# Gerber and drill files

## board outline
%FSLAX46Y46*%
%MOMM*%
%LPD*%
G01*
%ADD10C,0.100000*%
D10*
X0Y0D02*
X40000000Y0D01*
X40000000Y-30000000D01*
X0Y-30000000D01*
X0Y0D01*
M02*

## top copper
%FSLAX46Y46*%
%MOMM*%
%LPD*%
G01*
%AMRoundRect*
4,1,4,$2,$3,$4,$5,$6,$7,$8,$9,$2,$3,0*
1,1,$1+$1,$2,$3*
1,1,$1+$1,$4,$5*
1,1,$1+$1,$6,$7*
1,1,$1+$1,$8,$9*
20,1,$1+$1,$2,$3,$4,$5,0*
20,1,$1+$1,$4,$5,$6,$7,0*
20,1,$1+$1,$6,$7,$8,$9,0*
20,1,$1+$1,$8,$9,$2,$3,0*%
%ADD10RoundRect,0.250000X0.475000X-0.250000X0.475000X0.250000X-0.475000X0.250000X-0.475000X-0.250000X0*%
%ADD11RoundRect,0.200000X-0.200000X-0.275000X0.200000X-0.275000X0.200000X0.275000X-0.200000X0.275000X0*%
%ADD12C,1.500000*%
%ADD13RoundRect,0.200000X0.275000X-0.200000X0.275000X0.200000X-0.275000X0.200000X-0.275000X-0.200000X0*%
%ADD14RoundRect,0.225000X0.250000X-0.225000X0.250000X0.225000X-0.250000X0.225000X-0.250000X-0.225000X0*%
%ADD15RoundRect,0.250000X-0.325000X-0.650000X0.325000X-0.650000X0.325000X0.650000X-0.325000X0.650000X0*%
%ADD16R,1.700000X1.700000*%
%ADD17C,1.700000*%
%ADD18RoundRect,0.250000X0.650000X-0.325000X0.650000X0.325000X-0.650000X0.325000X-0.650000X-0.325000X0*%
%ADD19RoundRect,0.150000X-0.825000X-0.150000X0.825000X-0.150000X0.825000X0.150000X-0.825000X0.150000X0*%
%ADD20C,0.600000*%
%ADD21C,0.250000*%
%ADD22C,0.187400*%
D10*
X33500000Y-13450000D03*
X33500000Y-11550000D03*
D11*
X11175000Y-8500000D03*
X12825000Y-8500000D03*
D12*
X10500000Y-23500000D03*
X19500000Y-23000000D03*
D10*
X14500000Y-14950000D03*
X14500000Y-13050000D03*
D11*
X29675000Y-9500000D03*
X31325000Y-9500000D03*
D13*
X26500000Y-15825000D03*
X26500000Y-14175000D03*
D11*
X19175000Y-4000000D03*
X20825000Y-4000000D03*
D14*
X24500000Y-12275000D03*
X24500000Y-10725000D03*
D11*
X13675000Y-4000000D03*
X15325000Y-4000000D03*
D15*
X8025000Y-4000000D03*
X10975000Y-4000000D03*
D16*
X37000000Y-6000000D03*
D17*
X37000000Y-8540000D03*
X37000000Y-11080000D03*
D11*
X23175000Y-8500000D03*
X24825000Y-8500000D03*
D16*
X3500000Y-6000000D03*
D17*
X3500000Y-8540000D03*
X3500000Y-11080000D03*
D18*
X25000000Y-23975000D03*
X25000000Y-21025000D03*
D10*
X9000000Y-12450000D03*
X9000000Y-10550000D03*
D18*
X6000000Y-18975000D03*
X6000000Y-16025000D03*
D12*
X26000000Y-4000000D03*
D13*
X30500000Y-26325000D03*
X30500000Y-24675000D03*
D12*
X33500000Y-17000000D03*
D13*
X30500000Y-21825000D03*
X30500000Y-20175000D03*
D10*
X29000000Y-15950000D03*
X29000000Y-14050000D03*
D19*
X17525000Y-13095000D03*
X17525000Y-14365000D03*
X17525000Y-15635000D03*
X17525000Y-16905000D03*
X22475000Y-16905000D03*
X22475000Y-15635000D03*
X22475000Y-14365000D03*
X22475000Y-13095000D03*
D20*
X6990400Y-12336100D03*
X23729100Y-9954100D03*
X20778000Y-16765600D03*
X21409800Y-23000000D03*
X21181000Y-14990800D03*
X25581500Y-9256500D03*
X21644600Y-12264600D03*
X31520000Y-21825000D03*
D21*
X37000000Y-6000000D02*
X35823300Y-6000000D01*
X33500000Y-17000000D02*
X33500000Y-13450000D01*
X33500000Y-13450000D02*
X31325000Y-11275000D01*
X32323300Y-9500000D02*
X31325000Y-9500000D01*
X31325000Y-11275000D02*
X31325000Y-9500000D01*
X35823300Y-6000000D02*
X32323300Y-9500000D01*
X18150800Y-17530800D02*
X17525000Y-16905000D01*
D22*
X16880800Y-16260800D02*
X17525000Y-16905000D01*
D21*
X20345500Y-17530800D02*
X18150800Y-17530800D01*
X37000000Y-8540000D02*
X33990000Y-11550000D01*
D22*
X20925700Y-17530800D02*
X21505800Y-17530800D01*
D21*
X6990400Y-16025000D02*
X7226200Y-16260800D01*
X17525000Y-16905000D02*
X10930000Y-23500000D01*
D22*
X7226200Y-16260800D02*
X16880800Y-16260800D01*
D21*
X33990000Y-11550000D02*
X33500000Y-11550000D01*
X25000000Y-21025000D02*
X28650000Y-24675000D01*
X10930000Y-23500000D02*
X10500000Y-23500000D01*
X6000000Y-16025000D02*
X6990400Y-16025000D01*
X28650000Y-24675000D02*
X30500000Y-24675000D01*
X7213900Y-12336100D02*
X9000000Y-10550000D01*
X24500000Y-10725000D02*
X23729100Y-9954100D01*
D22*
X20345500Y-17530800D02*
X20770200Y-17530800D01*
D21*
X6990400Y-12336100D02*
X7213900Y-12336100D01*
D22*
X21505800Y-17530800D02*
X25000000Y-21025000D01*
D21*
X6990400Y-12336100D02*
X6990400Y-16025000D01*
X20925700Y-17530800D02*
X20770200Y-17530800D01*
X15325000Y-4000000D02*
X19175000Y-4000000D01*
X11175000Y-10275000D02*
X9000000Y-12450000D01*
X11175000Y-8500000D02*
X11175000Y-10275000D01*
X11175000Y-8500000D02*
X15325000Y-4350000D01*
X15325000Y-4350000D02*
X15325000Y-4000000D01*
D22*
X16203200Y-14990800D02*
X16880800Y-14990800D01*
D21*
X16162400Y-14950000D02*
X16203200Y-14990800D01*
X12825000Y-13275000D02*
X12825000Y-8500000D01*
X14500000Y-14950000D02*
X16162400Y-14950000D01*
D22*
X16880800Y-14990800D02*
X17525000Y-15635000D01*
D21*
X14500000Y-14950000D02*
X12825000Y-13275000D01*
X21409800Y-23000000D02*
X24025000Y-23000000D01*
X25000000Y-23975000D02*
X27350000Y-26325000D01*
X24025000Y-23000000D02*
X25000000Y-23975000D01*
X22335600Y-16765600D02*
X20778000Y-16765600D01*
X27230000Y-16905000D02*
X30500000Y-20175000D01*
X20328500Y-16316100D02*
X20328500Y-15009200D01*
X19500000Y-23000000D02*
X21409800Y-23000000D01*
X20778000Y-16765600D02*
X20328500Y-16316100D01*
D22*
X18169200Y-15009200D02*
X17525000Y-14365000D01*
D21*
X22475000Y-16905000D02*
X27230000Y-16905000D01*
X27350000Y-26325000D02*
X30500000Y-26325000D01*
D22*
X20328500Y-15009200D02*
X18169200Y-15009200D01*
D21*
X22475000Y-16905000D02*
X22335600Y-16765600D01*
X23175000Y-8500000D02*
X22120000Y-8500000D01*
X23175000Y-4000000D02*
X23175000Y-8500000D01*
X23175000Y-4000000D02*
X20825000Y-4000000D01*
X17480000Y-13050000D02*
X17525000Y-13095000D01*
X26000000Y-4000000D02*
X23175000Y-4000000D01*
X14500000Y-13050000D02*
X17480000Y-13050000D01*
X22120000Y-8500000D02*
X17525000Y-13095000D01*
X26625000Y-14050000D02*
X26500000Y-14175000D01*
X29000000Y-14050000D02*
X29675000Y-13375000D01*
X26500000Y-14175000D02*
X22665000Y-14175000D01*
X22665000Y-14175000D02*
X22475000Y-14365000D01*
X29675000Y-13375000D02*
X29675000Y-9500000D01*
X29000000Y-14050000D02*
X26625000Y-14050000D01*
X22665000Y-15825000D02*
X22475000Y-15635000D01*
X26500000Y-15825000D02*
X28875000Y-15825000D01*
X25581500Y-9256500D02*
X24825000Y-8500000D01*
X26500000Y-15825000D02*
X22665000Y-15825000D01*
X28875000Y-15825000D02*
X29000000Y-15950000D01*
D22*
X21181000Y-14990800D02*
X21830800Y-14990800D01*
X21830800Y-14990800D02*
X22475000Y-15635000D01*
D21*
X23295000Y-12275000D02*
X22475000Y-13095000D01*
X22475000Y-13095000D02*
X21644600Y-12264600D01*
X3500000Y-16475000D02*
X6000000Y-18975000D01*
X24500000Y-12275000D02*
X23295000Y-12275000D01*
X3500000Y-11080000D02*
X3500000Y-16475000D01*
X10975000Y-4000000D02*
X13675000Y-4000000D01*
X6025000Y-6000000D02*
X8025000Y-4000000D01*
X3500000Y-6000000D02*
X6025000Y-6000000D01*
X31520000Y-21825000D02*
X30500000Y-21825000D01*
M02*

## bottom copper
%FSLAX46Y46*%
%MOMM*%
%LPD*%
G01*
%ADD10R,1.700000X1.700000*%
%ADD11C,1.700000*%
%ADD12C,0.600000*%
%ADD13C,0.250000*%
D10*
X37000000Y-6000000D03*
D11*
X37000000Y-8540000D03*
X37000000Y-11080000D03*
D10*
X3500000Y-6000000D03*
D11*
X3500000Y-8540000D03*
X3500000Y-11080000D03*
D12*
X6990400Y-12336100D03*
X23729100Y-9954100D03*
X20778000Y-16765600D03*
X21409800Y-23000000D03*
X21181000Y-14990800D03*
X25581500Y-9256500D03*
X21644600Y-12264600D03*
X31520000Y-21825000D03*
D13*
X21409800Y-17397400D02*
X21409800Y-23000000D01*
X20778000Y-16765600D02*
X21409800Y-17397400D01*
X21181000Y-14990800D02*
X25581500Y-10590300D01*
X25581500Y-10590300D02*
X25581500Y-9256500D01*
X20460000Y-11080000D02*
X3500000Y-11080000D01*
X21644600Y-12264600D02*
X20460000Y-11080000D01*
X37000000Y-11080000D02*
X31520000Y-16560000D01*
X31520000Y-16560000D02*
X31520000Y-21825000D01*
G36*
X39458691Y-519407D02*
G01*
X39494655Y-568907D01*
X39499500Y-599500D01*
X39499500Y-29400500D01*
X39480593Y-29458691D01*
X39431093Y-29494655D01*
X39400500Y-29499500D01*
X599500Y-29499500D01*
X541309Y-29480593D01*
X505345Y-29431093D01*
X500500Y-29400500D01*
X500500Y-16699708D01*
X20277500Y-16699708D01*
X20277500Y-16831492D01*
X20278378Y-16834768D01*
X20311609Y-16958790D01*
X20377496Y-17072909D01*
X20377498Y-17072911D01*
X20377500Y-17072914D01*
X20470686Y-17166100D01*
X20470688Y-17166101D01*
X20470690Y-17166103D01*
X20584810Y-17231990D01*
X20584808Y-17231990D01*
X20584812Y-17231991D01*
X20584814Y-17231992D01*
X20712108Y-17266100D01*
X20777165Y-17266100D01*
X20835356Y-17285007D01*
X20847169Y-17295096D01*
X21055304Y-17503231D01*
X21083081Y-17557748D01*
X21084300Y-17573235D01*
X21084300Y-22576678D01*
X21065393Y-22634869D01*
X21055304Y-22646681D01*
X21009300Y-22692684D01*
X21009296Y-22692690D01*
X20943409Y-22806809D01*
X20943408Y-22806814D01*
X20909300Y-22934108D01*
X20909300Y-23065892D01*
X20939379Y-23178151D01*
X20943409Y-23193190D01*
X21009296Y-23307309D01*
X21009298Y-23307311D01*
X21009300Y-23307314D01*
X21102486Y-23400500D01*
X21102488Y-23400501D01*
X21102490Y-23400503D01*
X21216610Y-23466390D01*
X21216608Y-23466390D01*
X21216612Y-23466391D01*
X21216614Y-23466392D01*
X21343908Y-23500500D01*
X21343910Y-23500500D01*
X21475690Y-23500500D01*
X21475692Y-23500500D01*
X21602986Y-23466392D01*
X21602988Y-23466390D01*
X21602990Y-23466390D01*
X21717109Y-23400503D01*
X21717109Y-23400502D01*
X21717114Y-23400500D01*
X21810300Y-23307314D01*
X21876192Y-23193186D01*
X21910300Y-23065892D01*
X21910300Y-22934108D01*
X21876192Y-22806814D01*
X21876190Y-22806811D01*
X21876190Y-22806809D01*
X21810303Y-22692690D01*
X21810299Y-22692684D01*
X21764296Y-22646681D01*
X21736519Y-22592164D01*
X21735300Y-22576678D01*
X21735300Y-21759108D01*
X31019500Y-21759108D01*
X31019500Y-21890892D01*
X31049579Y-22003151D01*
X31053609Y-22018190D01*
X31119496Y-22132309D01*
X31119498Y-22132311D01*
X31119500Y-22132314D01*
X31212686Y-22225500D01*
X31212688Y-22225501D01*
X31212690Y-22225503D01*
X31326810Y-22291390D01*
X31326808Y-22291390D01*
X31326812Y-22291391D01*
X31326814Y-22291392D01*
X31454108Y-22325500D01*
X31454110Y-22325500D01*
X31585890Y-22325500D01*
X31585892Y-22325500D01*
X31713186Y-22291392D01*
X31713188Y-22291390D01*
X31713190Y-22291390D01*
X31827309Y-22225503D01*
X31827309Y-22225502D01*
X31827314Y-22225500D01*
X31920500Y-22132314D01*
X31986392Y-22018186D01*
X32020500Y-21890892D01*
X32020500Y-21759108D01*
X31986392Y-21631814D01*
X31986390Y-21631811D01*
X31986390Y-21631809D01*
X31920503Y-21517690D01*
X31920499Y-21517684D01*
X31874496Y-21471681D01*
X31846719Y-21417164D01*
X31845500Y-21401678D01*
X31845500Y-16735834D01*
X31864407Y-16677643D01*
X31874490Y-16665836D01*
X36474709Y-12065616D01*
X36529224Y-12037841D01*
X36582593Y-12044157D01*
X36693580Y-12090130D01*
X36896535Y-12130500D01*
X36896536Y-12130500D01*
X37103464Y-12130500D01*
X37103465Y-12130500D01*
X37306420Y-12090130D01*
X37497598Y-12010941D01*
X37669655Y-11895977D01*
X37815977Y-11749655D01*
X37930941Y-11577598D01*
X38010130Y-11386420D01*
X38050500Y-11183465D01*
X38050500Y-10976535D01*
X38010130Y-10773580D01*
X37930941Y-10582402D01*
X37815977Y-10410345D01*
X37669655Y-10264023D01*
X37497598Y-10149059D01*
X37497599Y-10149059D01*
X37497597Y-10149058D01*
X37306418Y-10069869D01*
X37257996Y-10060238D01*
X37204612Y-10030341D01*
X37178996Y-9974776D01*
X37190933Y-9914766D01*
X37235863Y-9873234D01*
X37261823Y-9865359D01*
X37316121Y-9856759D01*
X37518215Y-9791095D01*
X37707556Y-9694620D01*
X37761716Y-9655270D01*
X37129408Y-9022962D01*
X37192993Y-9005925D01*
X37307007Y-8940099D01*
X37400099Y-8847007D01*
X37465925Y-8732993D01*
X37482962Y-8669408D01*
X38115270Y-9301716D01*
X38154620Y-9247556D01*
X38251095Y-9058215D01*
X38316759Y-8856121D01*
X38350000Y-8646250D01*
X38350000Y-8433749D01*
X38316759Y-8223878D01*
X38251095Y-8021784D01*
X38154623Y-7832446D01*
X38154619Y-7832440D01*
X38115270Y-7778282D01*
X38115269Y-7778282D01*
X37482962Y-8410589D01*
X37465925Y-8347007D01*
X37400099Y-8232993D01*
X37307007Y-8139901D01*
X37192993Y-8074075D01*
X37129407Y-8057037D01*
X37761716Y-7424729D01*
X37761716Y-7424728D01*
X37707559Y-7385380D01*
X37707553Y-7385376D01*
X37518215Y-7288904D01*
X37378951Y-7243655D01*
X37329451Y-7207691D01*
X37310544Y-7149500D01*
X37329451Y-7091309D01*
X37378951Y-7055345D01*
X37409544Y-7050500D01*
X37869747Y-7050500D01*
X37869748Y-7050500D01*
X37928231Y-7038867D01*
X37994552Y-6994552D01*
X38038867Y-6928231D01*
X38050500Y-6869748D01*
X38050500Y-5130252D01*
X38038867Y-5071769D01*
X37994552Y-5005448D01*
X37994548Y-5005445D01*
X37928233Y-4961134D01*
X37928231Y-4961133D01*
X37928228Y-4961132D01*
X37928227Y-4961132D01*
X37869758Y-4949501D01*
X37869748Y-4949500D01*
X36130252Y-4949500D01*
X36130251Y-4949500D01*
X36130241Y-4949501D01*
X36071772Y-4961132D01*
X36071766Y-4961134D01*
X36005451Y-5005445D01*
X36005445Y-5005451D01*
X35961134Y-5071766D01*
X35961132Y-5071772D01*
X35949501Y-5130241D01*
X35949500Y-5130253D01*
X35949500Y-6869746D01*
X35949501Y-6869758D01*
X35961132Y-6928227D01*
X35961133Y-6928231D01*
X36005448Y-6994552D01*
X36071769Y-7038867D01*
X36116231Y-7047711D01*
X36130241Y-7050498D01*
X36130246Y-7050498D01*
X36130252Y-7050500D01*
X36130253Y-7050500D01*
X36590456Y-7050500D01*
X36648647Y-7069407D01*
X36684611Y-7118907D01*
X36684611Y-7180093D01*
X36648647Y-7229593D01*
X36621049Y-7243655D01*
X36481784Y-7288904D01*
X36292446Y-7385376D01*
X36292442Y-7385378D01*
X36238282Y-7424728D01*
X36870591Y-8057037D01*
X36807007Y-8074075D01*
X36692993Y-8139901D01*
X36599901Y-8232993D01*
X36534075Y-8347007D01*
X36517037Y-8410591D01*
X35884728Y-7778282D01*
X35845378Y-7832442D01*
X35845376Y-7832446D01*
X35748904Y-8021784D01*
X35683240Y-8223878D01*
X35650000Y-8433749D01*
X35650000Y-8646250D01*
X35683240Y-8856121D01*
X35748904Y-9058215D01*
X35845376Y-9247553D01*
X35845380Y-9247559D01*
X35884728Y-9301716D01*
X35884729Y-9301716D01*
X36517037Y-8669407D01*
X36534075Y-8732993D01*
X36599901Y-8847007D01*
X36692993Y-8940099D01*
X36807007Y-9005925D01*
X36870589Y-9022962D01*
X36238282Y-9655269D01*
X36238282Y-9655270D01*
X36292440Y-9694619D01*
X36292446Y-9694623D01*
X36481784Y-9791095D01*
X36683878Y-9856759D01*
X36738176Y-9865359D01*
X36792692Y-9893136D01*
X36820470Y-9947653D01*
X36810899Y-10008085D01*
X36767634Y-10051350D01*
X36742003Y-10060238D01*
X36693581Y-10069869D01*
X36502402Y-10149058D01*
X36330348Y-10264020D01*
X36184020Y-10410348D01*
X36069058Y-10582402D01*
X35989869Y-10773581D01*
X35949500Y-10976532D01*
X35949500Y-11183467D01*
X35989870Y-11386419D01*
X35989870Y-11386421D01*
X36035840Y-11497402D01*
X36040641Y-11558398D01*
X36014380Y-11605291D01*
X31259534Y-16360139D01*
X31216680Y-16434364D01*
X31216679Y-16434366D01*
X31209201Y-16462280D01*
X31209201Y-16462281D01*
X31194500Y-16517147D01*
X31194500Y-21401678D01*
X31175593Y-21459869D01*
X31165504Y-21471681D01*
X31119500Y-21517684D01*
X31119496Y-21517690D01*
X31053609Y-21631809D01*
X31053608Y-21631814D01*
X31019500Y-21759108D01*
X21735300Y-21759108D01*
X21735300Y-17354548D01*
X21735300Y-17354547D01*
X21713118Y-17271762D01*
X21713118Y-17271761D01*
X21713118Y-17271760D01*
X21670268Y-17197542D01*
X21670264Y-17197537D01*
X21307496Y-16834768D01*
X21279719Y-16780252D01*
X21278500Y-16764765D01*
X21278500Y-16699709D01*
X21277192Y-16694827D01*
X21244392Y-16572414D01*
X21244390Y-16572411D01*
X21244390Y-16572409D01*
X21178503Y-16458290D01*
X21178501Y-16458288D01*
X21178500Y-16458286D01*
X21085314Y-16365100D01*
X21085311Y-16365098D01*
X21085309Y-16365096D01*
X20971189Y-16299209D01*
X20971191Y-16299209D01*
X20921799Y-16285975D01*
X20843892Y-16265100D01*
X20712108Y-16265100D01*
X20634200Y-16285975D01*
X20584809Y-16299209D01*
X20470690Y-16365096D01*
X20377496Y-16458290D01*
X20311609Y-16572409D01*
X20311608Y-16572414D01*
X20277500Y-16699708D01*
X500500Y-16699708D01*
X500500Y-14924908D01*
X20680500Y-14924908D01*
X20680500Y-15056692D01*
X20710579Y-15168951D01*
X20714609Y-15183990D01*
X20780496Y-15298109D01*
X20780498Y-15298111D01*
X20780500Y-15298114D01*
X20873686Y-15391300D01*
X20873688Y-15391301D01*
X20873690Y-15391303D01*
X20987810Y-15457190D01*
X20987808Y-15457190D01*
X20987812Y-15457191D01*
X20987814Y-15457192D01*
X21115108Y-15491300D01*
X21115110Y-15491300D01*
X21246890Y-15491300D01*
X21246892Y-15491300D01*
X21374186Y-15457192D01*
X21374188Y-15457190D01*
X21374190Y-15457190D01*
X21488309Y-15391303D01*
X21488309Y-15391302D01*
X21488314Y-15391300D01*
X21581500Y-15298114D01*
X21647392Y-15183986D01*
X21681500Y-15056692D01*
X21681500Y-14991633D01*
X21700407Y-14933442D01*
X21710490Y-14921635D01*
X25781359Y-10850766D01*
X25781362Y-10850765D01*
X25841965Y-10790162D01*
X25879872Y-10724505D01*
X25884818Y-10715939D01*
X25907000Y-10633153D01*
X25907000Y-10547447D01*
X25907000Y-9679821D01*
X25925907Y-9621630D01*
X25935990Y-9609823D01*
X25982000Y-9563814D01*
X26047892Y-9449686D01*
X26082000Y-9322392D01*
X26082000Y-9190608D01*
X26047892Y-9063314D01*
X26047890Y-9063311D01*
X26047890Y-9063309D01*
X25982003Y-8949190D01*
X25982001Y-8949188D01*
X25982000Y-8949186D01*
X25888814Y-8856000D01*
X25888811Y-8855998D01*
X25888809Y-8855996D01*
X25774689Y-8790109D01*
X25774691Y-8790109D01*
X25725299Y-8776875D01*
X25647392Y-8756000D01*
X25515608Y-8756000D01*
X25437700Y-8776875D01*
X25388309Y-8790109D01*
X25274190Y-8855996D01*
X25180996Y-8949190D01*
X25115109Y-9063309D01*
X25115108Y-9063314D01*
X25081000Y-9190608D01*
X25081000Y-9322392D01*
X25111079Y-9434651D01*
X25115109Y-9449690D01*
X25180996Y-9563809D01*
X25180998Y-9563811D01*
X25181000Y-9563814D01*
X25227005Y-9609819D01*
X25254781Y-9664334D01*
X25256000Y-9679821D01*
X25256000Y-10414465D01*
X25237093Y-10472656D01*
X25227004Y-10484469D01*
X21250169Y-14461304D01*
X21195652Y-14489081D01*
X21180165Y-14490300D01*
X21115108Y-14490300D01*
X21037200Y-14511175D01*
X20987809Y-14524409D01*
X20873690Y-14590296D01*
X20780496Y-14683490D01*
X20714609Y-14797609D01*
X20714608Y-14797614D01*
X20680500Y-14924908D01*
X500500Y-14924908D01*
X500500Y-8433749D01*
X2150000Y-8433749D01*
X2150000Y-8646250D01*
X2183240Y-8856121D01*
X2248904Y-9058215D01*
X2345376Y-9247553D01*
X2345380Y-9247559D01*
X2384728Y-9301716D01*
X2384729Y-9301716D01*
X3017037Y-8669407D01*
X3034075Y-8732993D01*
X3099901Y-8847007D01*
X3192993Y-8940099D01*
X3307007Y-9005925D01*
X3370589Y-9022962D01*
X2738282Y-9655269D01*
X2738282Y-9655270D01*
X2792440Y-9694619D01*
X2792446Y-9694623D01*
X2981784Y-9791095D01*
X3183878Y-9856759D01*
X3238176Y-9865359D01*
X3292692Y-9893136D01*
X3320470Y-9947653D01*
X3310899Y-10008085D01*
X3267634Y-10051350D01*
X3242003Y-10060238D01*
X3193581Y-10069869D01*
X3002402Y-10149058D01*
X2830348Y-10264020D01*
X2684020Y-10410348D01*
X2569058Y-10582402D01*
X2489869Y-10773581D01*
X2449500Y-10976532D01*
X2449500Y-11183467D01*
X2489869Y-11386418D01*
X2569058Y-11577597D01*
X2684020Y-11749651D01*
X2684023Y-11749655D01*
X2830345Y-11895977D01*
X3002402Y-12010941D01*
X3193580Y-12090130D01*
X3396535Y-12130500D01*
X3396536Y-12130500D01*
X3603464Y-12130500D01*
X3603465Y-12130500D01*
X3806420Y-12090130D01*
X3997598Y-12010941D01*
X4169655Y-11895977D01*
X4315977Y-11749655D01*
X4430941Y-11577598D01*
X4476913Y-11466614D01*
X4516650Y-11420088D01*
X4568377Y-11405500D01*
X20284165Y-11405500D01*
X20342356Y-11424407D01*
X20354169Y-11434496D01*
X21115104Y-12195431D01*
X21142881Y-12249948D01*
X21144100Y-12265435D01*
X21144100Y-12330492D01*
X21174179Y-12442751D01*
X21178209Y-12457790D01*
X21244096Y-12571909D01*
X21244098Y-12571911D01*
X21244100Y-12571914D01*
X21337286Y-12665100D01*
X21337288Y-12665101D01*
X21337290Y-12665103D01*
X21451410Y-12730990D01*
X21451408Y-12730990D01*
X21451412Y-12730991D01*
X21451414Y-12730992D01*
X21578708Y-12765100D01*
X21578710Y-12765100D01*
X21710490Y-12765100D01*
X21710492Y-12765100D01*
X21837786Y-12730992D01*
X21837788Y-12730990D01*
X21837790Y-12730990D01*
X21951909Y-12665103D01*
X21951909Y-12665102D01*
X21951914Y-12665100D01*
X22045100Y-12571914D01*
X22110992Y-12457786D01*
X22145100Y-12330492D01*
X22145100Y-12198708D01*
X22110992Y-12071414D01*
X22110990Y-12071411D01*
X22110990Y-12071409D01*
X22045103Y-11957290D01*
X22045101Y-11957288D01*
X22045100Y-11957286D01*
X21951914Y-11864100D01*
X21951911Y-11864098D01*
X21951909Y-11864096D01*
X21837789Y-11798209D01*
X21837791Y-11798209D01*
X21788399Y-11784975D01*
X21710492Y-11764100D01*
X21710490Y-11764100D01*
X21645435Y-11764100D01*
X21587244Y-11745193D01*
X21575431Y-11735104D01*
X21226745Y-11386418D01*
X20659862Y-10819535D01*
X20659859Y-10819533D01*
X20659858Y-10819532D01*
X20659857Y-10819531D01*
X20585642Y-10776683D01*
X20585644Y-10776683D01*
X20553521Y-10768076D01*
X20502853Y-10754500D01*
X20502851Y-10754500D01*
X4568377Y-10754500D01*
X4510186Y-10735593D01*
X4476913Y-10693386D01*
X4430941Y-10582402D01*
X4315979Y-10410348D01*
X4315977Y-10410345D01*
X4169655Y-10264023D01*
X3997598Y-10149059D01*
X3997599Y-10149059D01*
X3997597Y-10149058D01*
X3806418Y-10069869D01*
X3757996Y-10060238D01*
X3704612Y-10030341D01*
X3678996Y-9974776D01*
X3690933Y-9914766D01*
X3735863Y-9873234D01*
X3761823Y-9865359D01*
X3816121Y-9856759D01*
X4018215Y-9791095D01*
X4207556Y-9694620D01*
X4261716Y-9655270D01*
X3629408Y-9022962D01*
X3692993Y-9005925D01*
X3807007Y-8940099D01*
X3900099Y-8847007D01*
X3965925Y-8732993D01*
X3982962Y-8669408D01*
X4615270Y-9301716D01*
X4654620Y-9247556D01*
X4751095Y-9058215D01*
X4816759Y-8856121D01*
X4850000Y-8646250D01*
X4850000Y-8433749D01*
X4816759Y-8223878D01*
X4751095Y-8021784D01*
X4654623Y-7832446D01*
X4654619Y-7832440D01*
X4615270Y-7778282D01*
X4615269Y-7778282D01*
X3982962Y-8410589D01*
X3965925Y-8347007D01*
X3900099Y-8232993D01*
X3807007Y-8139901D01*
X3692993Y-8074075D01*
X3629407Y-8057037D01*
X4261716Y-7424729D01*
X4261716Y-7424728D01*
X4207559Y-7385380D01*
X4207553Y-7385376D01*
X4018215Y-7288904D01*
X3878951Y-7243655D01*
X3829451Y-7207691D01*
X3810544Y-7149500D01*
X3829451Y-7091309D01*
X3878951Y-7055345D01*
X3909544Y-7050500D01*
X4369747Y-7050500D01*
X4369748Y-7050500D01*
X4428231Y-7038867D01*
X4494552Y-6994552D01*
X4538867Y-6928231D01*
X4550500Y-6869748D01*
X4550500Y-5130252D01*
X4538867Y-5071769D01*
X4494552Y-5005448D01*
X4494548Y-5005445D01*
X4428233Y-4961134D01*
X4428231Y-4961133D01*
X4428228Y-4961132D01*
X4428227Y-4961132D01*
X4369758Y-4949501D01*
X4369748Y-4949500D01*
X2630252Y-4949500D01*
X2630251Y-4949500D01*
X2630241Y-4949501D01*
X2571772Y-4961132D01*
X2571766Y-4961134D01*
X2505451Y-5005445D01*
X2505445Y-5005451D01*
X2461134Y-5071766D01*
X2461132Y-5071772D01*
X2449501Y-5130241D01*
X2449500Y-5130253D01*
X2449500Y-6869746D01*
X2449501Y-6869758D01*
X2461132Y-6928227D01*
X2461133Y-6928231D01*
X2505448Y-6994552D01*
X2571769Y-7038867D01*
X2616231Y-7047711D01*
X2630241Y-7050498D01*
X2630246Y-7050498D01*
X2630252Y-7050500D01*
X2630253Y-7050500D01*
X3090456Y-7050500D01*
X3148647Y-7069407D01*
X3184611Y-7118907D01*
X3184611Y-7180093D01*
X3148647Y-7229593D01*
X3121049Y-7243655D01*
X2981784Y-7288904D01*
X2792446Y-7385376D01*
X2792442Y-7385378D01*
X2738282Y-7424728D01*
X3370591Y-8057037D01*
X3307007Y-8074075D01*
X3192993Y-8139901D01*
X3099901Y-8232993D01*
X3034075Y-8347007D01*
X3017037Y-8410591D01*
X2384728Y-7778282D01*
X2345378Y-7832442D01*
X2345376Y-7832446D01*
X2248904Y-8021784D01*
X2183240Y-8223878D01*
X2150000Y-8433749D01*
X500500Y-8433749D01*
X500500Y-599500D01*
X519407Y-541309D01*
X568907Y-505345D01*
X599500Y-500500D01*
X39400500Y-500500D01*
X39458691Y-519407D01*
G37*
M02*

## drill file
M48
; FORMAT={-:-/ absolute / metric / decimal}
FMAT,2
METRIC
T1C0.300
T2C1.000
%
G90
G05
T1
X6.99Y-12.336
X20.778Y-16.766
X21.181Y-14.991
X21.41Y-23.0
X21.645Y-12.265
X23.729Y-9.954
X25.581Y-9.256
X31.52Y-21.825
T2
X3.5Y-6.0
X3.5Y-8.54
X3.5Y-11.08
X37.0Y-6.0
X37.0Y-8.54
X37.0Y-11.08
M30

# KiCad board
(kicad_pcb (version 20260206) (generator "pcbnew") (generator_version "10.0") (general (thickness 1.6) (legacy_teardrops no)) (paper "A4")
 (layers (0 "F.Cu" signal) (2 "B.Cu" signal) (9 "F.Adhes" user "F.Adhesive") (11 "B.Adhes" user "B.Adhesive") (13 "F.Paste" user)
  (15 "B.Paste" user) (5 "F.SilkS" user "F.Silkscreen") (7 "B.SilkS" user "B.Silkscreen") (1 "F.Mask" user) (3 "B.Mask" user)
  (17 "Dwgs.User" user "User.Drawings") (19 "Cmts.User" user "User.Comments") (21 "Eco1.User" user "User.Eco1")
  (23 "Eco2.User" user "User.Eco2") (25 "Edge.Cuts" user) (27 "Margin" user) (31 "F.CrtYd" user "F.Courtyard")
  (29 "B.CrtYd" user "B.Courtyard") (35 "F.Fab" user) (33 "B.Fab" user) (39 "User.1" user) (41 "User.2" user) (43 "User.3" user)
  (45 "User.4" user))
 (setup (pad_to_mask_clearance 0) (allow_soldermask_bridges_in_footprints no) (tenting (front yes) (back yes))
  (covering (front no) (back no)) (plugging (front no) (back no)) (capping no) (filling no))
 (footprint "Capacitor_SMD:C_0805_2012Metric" (layer "F.Cu") (at 33.5 12.5 90)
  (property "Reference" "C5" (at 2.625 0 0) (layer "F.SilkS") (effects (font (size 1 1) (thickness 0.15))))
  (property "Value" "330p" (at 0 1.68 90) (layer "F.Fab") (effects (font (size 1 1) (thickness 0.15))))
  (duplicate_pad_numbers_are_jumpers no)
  (pad "1" smd roundrect (at -0.95 0 90) (size 1 1.45) (layers "F.Cu" "F.Mask" "F.Paste") (roundrect_rratio 0.25) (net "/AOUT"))
  (pad "2" smd roundrect (at 0.95 0 90) (size 1 1.45) (layers "F.Cu" "F.Mask" "F.Paste") (roundrect_rratio 0.25) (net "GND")))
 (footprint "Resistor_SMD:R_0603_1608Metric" (layer "F.Cu") (at 12 8.5)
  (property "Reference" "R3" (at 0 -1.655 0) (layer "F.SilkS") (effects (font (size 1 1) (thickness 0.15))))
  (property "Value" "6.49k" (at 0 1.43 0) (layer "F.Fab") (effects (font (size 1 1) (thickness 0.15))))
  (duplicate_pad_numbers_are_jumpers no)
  (pad "1" smd roundrect (at -0.825 0) (size 0.8 0.95) (layers "F.Cu" "F.Mask" "F.Paste") (roundrect_rratio 0.25) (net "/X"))
  (pad "2" smd roundrect (at 0.825 0) (size 0.8 0.95) (layers "F.Cu" "F.Mask" "F.Paste") (roundrect_rratio 0.25) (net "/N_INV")))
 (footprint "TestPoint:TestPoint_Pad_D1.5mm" (layer "F.Cu") (at 10.5 23.5)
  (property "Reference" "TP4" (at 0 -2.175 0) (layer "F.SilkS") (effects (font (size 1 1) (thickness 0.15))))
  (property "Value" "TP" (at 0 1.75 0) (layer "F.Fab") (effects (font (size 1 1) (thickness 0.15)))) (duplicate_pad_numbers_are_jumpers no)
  (pad "1" smd circle (at 0 0) (size 1.5 1.5) (layers "F.Cu" "F.Mask") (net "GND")))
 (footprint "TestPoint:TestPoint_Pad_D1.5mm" (layer "F.Cu") (at 19.5 23)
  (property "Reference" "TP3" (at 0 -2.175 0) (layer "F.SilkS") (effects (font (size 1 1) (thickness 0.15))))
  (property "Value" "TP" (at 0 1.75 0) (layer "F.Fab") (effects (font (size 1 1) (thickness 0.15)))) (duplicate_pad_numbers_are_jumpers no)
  (pad "1" smd circle (at 0 0) (size 1.5 1.5) (layers "F.Cu" "F.Mask") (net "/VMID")))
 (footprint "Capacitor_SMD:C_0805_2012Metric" (layer "F.Cu") (at 14.5 14 90)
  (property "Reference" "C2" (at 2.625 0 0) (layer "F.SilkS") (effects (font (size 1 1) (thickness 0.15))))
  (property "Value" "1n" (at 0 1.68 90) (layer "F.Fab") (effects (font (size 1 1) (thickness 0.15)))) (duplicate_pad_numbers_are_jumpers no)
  (pad "1" smd roundrect (at -0.95 0 90) (size 1 1.45) (layers "F.Cu" "F.Mask" "F.Paste") (roundrect_rratio 0.25) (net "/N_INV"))
  (pad "2" smd roundrect (at 0.95 0 90) (size 1 1.45) (layers "F.Cu" "F.Mask" "F.Paste") (roundrect_rratio 0.25) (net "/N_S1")))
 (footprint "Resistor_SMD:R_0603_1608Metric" (layer "F.Cu") (at 30.5 9.5)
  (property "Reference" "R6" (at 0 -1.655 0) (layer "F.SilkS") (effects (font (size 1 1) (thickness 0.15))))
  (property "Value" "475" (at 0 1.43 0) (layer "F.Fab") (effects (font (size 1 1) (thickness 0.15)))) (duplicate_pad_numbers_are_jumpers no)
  (pad "1" smd roundrect (at -0.825 0) (size 0.8 0.95) (layers "F.Cu" "F.Mask" "F.Paste") (roundrect_rratio 0.25) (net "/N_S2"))
  (pad "2" smd roundrect (at 0.825 0) (size 0.8 0.95) (layers "F.Cu" "F.Mask" "F.Paste") (roundrect_rratio 0.25) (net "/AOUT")))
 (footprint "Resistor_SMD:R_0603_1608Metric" (layer "F.Cu") (at 26.5 15 90)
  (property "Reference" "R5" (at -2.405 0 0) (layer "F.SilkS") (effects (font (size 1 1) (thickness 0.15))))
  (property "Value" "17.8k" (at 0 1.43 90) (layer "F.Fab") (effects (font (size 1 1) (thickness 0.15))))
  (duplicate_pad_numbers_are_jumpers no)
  (pad "1" smd roundrect (at -0.825 0 90) (size 0.8 0.95) (layers "F.Cu" "F.Mask" "F.Paste") (roundrect_rratio 0.25) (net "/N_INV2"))
  (pad "2" smd roundrect (at 0.825 0 90) (size 0.8 0.95) (layers "F.Cu" "F.Mask" "F.Paste") (roundrect_rratio 0.25) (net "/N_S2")))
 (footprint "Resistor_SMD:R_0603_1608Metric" (layer "F.Cu") (at 20 4)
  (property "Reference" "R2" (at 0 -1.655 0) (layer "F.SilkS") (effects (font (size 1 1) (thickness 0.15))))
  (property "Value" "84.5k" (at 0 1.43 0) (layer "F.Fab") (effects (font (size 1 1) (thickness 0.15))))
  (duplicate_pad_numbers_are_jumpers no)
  (pad "1" smd roundrect (at -0.825 0) (size 0.8 0.95) (layers "F.Cu" "F.Mask" "F.Paste") (roundrect_rratio 0.25) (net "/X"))
  (pad "2" smd roundrect (at 0.825 0) (size 0.8 0.95) (layers "F.Cu" "F.Mask" "F.Paste") (roundrect_rratio 0.25) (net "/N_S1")))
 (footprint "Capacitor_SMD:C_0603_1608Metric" (layer "F.Cu") (at 24.5 11.5 90)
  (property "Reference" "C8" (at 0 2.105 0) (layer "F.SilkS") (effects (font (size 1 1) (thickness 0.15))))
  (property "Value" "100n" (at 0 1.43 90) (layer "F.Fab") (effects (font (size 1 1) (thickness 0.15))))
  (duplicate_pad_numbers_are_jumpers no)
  (pad "1" smd roundrect (at -0.775 0 90) (size 0.9 0.95) (layers "F.Cu" "F.Mask" "F.Paste") (roundrect_rratio 0.25) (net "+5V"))
  (pad "2" smd roundrect (at 0.775 0 90) (size 0.9 0.95) (layers "F.Cu" "F.Mask" "F.Paste") (roundrect_rratio 0.25) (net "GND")))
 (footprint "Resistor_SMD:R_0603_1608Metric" (layer "F.Cu") (at 14.5 4)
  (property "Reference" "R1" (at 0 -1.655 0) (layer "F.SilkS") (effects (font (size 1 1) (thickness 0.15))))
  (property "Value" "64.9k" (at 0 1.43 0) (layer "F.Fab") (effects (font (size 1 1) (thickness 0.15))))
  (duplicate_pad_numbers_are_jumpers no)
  (pad "1" smd roundrect (at -0.825 0) (size 0.8 0.95) (layers "F.Cu" "F.Mask" "F.Paste") (roundrect_rratio 0.25) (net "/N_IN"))
  (pad "2" smd roundrect (at 0.825 0) (size 0.8 0.95) (layers "F.Cu" "F.Mask" "F.Paste") (roundrect_rratio 0.25) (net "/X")))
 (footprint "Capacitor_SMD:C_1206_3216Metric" (layer "F.Cu") (at 9.5 4)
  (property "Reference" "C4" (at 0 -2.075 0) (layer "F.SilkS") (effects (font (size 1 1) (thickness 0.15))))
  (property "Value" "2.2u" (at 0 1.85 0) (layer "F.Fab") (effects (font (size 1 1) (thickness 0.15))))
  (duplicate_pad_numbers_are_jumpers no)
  (pad "1" smd roundrect (at -1.475 0) (size 1.15 1.8) (layers "F.Cu" "F.Mask" "F.Paste") (roundrect_rratio 0.217391) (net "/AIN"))
  (pad "2" smd roundrect (at 1.475 0) (size 1.15 1.8) (layers "F.Cu" "F.Mask" "F.Paste") (roundrect_rratio 0.217391) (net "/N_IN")))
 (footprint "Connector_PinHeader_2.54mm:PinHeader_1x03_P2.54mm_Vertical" (layer "F.Cu") (at 37 6)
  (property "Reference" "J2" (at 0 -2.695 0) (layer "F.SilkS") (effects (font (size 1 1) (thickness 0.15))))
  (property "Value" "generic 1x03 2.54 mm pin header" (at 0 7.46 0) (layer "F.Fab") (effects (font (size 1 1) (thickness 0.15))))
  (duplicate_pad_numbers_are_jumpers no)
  (pad "1" thru_hole rect (at 0 0) (size 1.7 1.7) (drill 1) (layers "*.Cu" "*.Mask") (remove_unused_layers no) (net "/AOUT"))
  (pad "2" thru_hole circle (at 0 2.54) (size 1.7 1.7) (drill 1) (layers "*.Cu" "*.Mask") (remove_unused_layers no) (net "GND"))
  (pad "3" thru_hole circle (at 0 5.08) (size 1.7 1.7) (drill 1) (layers "*.Cu" "*.Mask") (remove_unused_layers no) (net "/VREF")))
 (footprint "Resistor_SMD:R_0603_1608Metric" (layer "F.Cu") (at 24 8.5)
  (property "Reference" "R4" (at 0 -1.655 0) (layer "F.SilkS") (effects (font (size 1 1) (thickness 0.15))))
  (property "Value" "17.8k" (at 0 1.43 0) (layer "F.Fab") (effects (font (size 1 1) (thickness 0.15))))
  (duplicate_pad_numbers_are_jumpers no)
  (pad "1" smd roundrect (at -0.825 0) (size 0.8 0.95) (layers "F.Cu" "F.Mask" "F.Paste") (roundrect_rratio 0.25) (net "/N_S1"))
  (pad "2" smd roundrect (at 0.825 0) (size 0.8 0.95) (layers "F.Cu" "F.Mask" "F.Paste") (roundrect_rratio 0.25) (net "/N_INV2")))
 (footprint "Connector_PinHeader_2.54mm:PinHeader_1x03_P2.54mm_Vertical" (layer "F.Cu") (at 3.5 6)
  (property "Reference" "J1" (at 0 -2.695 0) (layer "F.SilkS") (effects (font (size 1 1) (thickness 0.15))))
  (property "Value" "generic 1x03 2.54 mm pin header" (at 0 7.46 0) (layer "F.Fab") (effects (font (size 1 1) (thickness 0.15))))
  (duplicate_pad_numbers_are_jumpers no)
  (pad "1" thru_hole rect (at 0 0) (size 1.7 1.7) (drill 1) (layers "*.Cu" "*.Mask") (remove_unused_layers no) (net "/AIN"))
  (pad "2" thru_hole circle (at 0 2.54) (size 1.7 1.7) (drill 1) (layers "*.Cu" "*.Mask") (remove_unused_layers no) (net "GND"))
  (pad "3" thru_hole circle (at 0 5.08) (size 1.7 1.7) (drill 1) (layers "*.Cu" "*.Mask") (remove_unused_layers no) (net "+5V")))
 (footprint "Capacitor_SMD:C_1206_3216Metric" (layer "F.Cu") (at 25 22.5 90)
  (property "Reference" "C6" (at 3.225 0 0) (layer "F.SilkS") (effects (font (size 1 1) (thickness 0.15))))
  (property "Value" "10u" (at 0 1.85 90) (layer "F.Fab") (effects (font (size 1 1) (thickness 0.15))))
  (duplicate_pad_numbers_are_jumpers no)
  (pad "1" smd roundrect (at -1.475 0 90) (size 1.15 1.8) (layers "F.Cu" "F.Mask" "F.Paste") (roundrect_rratio 0.217391) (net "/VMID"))
  (pad "2" smd roundrect (at 1.475 0 90) (size 1.15 1.8) (layers "F.Cu" "F.Mask" "F.Paste") (roundrect_rratio 0.217391) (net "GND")))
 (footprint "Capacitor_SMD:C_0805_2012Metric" (layer "F.Cu") (at 9 11.5 90)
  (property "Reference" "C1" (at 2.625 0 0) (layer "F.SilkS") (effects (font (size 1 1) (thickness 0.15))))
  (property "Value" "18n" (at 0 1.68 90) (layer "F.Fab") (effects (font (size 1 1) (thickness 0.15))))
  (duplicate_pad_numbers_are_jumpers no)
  (pad "1" smd roundrect (at -0.95 0 90) (size 1 1.45) (layers "F.Cu" "F.Mask" "F.Paste") (roundrect_rratio 0.25) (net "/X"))
  (pad "2" smd roundrect (at 0.95 0 90) (size 1 1.45) (layers "F.Cu" "F.Mask" "F.Paste") (roundrect_rratio 0.25) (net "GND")))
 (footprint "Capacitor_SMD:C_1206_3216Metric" (layer "F.Cu") (at 6 17.5 90)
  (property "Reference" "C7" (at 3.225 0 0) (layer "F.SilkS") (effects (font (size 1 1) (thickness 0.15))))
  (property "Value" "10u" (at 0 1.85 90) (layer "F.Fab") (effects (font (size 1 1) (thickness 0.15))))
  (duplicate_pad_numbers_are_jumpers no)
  (pad "1" smd roundrect (at -1.475 0 90) (size 1.15 1.8) (layers "F.Cu" "F.Mask" "F.Paste") (roundrect_rratio 0.217391) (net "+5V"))
  (pad "2" smd roundrect (at 1.475 0 90) (size 1.15 1.8) (layers "F.Cu" "F.Mask" "F.Paste") (roundrect_rratio 0.217391) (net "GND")))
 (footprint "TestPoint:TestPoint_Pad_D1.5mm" (layer "F.Cu") (at 26 4)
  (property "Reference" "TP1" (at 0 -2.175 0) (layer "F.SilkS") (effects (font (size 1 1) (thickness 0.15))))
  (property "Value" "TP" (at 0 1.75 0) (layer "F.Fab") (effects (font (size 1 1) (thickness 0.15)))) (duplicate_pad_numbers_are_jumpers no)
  (pad "1" smd circle (at 0 0) (size 1.5 1.5) (layers "F.Cu" "F.Mask") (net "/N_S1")))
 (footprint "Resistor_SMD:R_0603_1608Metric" (layer "F.Cu") (at 30.5 25.5 90)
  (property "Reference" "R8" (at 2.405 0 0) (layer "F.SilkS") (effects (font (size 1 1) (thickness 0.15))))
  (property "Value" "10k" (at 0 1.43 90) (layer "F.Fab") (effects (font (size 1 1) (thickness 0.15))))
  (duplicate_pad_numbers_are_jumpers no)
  (pad "1" smd roundrect (at -0.825 0 90) (size 0.8 0.95) (layers "F.Cu" "F.Mask" "F.Paste") (roundrect_rratio 0.25) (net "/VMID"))
  (pad "2" smd roundrect (at 0.825 0 90) (size 0.8 0.95) (layers "F.Cu" "F.Mask" "F.Paste") (roundrect_rratio 0.25) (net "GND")))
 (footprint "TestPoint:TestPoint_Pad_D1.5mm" (layer "F.Cu") (at 33.5 17)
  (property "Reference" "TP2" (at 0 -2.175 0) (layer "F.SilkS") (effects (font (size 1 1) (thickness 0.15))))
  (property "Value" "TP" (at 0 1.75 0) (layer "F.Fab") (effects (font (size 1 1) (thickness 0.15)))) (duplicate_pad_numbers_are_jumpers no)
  (pad "1" smd circle (at 0 0) (size 1.5 1.5) (layers "F.Cu" "F.Mask") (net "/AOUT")))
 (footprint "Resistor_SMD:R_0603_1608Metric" (layer "F.Cu") (at 30.5 21 90)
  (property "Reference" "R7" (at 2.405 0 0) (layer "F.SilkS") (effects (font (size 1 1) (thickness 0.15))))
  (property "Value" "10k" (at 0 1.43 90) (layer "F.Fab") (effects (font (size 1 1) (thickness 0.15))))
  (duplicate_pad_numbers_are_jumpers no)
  (pad "1" smd roundrect (at -0.825 0 90) (size 0.8 0.95) (layers "F.Cu" "F.Mask" "F.Paste") (roundrect_rratio 0.25) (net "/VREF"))
  (pad "2" smd roundrect (at 0.825 0 90) (size 0.8 0.95) (layers "F.Cu" "F.Mask" "F.Paste") (roundrect_rratio 0.25) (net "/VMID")))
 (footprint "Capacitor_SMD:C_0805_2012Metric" (layer "F.Cu") (at 29 15 90)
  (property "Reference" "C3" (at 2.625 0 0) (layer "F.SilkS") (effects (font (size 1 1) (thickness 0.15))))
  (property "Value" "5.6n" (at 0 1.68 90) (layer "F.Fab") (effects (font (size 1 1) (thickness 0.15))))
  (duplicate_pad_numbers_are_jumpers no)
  (pad "1" smd roundrect (at -0.95 0 90) (size 1 1.45) (layers "F.Cu" "F.Mask" "F.Paste") (roundrect_rratio 0.25) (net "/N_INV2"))
  (pad "2" smd roundrect (at 0.95 0 90) (size 1 1.45) (layers "F.Cu" "F.Mask" "F.Paste") (roundrect_rratio 0.25) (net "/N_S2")))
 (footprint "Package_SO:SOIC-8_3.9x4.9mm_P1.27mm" (layer "F.Cu") (at 20 15)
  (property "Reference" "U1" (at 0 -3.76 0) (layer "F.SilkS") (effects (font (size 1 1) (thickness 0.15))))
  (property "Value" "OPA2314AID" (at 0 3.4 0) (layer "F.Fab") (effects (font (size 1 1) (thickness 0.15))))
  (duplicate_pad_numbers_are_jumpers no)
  (pad "1" smd roundrect (at -2.475 -1.905) (size 1.95 0.6) (layers "F.Cu" "F.Mask" "F.Paste") (roundrect_rratio 0.25) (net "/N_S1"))
  (pad "2" smd roundrect (at -2.475 -0.635) (size 1.95 0.6) (layers "F.Cu" "F.Mask" "F.Paste") (roundrect_rratio 0.25) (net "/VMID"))
  (pad "3" smd roundrect (at -2.475 0.635) (size 1.95 0.6) (layers "F.Cu" "F.Mask" "F.Paste") (roundrect_rratio 0.25) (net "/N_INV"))
  (pad "4" smd roundrect (at -2.475 1.905) (size 1.95 0.6) (layers "F.Cu" "F.Mask" "F.Paste") (roundrect_rratio 0.25) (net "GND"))
  (pad "5" smd roundrect (at 2.475 1.905) (size 1.95 0.6) (layers "F.Cu" "F.Mask" "F.Paste") (roundrect_rratio 0.25) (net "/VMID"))
  (pad "6" smd roundrect (at 2.475 0.635) (size 1.95 0.6) (layers "F.Cu" "F.Mask" "F.Paste") (roundrect_rratio 0.25) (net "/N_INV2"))
  (pad "7" smd roundrect (at 2.475 -0.635) (size 1.95 0.6) (layers "F.Cu" "F.Mask" "F.Paste") (roundrect_rratio 0.25) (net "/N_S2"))
  (pad "8" smd roundrect (at 2.475 -1.905) (size 1.95 0.6) (layers "F.Cu" "F.Mask" "F.Paste") (roundrect_rratio 0.25) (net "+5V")))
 (gr_rect (start 0 0) (end 40 30) (stroke (width 0.1) (type default)) (fill no) (layer "Edge.Cuts"))
 (segment (start 37 6) (end 35.8233 6) (width 0.25) (layer "F.Cu") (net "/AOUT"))
 (segment (start 33.5 17) (end 33.5 13.45) (width 0.25) (layer "F.Cu") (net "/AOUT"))
 (segment (start 33.5 13.45) (end 31.325 11.275) (width 0.25) (layer "F.Cu") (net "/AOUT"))
 (segment (start 32.3233 9.5) (end 31.325 9.5) (width 0.25) (layer "F.Cu") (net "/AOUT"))
 (segment (start 31.325 11.275) (end 31.325 9.5) (width 0.25) (layer "F.Cu") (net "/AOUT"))
 (segment (start 35.8233 6) (end 32.3233 9.5) (width 0.25) (layer "F.Cu") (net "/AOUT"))
 (segment (start 18.1508 17.5308) (end 17.525 16.905) (width 0.25) (layer "F.Cu") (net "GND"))
 (segment (start 16.8808 16.2608) (end 17.525 16.905) (width 0.1874) (layer "F.Cu") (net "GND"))
 (segment (start 20.3455 17.5308) (end 18.1508 17.5308) (width 0.25) (layer "F.Cu") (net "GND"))
 (segment (start 37 8.54) (end 33.99 11.55) (width 0.25) (layer "F.Cu") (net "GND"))
 (segment (start 20.9257 17.5308) (end 21.5058 17.5308) (width 0.1874) (layer "F.Cu") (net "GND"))
 (segment (start 6.9904 16.025) (end 7.2262 16.2608) (width 0.25) (layer "F.Cu") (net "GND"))
 (segment (start 17.525 16.905) (end 10.93 23.5) (width 0.25) (layer "F.Cu") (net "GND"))
 (segment (start 7.2262 16.2608) (end 16.8808 16.2608) (width 0.1874) (layer "F.Cu") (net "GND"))
 (segment (start 33.99 11.55) (end 33.5 11.55) (width 0.25) (layer "F.Cu") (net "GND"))
 (segment (start 25 21.025) (end 28.65 24.675) (width 0.25) (layer "F.Cu") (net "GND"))
 (segment (start 10.93 23.5) (end 10.5 23.5) (width 0.25) (layer "F.Cu") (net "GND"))
 (segment (start 6 16.025) (end 6.9904 16.025) (width 0.25) (layer "F.Cu") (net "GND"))
 (segment (start 28.65 24.675) (end 30.5 24.675) (width 0.25) (layer "F.Cu") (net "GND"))
 (segment (start 7.2139 12.3361) (end 9 10.55) (width 0.25) (layer "F.Cu") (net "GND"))
 (segment (start 24.5 10.725) (end 23.7291 9.9541) (width 0.25) (layer "F.Cu") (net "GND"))
 (segment (start 20.3455 17.5308) (end 20.7702 17.5308) (width 0.1874) (layer "F.Cu") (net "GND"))
 (segment (start 6.9904 12.3361) (end 7.2139 12.3361) (width 0.25) (layer "F.Cu") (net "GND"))
 (segment (start 21.5058 17.5308) (end 25 21.025) (width 0.1874) (layer "F.Cu") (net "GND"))
 (segment (start 6.9904 12.3361) (end 6.9904 16.025) (width 0.25) (layer "F.Cu") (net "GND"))
 (segment (start 20.9257 17.5308) (end 20.7702 17.5308) (width 0.25) (layer "F.Cu") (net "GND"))
 (via (at 6.9904 12.3361) (size 0.6) (drill 0.3) (layers "F.Cu" "B.Cu") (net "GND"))
 (via (at 23.7291 9.9541) (size 0.6) (drill 0.3) (layers "F.Cu" "B.Cu") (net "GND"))
 (segment (start 15.325 4) (end 19.175 4) (width 0.25) (layer "F.Cu") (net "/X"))
 (segment (start 11.175 10.275) (end 9 12.45) (width 0.25) (layer "F.Cu") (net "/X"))
 (segment (start 11.175 8.5) (end 11.175 10.275) (width 0.25) (layer "F.Cu") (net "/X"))
 (segment (start 11.175 8.5) (end 15.325 4.35) (width 0.25) (layer "F.Cu") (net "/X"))
 (segment (start 15.325 4.35) (end 15.325 4) (width 0.25) (layer "F.Cu") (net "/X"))
 (segment (start 16.2032 14.9908) (end 16.8808 14.9908) (width 0.1874) (layer "F.Cu") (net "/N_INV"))
 (segment (start 16.1624 14.95) (end 16.2032 14.9908) (width 0.25) (layer "F.Cu") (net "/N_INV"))
 (segment (start 12.825 13.275) (end 12.825 8.5) (width 0.25) (layer "F.Cu") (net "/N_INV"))
 (segment (start 14.5 14.95) (end 16.1624 14.95) (width 0.25) (layer "F.Cu") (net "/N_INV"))
 (segment (start 16.8808 14.9908) (end 17.525 15.635) (width 0.1874) (layer "F.Cu") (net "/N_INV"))
 (segment (start 14.5 14.95) (end 12.825 13.275) (width 0.25) (layer "F.Cu") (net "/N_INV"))
 (segment (start 21.4098 23) (end 24.025 23) (width 0.25) (layer "F.Cu") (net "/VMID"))
 (segment (start 25 23.975) (end 27.35 26.325) (width 0.25) (layer "F.Cu") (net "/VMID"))
 (segment (start 24.025 23) (end 25 23.975) (width 0.25) (layer "F.Cu") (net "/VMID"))
 (segment (start 22.3356 16.7656) (end 20.778 16.7656) (width 0.25) (layer "F.Cu") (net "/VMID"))
 (segment (start 27.23 16.905) (end 30.5 20.175) (width 0.25) (layer "F.Cu") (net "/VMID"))
 (segment (start 20.3285 16.3161) (end 20.3285 15.0092) (width 0.25) (layer "F.Cu") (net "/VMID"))
 (segment (start 19.5 23) (end 21.4098 23) (width 0.25) (layer "F.Cu") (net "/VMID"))
 (segment (start 20.778 16.7656) (end 20.3285 16.3161) (width 0.25) (layer "F.Cu") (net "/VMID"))
 (segment (start 18.1692 15.0092) (end 17.525 14.365) (width 0.1874) (layer "F.Cu") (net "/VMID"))
 (segment (start 22.475 16.905) (end 27.23 16.905) (width 0.25) (layer "F.Cu") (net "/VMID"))
 (segment (start 27.35 26.325) (end 30.5 26.325) (width 0.25) (layer "F.Cu") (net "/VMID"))
 (segment (start 20.3285 15.0092) (end 18.1692 15.0092) (width 0.1874) (layer "F.Cu") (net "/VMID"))
 (segment (start 22.475 16.905) (end 22.3356 16.7656) (width 0.25) (layer "F.Cu") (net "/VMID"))
 (via (at 20.778 16.7656) (size 0.6) (drill 0.3) (layers "F.Cu" "B.Cu") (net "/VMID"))
 (via (at 21.4098 23) (size 0.6) (drill 0.3) (layers "F.Cu" "B.Cu") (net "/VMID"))
 (segment (start 21.4098 17.3974) (end 21.4098 23) (width 0.25) (layer "B.Cu") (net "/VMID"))
 (segment (start 20.778 16.7656) (end 21.4098 17.3974) (width 0.25) (layer "B.Cu") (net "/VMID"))
 (segment (start 23.175 8.5) (end 22.12 8.5) (width 0.25) (layer "F.Cu") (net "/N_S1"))
 (segment (start 23.175 4) (end 23.175 8.5) (width 0.25) (layer "F.Cu") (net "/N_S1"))
 (segment (start 23.175 4) (end 20.825 4) (width 0.25) (layer "F.Cu") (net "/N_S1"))
 (segment (start 17.48 13.05) (end 17.525 13.095) (width 0.25) (layer "F.Cu") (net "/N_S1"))
 (segment (start 26 4) (end 23.175 4) (width 0.25) (layer "F.Cu") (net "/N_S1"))
 (segment (start 14.5 13.05) (end 17.48 13.05) (width 0.25) (layer "F.Cu") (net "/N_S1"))
 (segment (start 22.12 8.5) (end 17.525 13.095) (width 0.25) (layer "F.Cu") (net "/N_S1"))
 (segment (start 26.625 14.05) (end 26.5 14.175) (width 0.25) (layer "F.Cu") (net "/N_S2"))
 (segment (start 29 14.05) (end 29.675 13.375) (width 0.25) (layer "F.Cu") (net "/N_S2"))
 (segment (start 26.5 14.175) (end 22.665 14.175) (width 0.25) (layer "F.Cu") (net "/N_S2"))
 (segment (start 22.665 14.175) (end 22.475 14.365) (width 0.25) (layer "F.Cu") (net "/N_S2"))
 (segment (start 29.675 13.375) (end 29.675 9.5) (width 0.25) (layer "F.Cu") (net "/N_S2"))
 (segment (start 29 14.05) (end 26.625 14.05) (width 0.25) (layer "F.Cu") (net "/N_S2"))
 (segment (start 22.665 15.825) (end 22.475 15.635) (width 0.25) (layer "F.Cu") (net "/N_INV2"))
 (segment (start 26.5 15.825) (end 28.875 15.825) (width 0.25) (layer "F.Cu") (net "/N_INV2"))
 (segment (start 25.5815 9.2565) (end 24.825 8.5) (width 0.25) (layer "F.Cu") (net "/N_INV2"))
 (segment (start 26.5 15.825) (end 22.665 15.825) (width 0.25) (layer "F.Cu") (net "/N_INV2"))
 (segment (start 28.875 15.825) (end 29 15.95) (width 0.25) (layer "F.Cu") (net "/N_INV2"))
 (segment (start 21.181 14.9908) (end 21.8308 14.9908) (width 0.1874) (layer "F.Cu") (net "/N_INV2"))
 (segment (start 21.8308 14.9908) (end 22.475 15.635) (width 0.1874) (layer "F.Cu") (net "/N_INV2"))
 (via (at 21.181 14.9908) (size 0.6) (drill 0.3) (layers "F.Cu" "B.Cu") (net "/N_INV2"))
 (via (at 25.5815 9.2565) (size 0.6) (drill 0.3) (layers "F.Cu" "B.Cu") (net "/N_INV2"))
 (segment (start 21.181 14.9908) (end 25.5815 10.5903) (width 0.25) (layer "B.Cu") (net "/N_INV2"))
 (segment (start 25.5815 10.5903) (end 25.5815 9.2565) (width 0.25) (layer "B.Cu") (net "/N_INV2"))
 (segment (start 23.295 12.275) (end 22.475 13.095) (width 0.25) (layer "F.Cu") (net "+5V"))
 (segment (start 22.475 13.095) (end 21.6446 12.2646) (width 0.25) (layer "F.Cu") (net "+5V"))
 (segment (start 3.5 16.475) (end 6 18.975) (width 0.25) (layer "F.Cu") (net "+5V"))
 (segment (start 24.5 12.275) (end 23.295 12.275) (width 0.25) (layer "F.Cu") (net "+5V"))
 (segment (start 3.5 11.08) (end 3.5 16.475) (width 0.25) (layer "F.Cu") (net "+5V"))
 (via (at 21.6446 12.2646) (size 0.6) (drill 0.3) (layers "F.Cu" "B.Cu") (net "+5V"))
 (segment (start 20.46 11.08) (end 3.5 11.08) (width 0.25) (layer "B.Cu") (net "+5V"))
 (segment (start 21.6446 12.2646) (end 20.46 11.08) (width 0.25) (layer "B.Cu") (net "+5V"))
 (segment (start 10.975 4) (end 13.675 4) (width 0.25) (layer "F.Cu") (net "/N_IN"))
 (segment (start 6.025 6) (end 8.025 4) (width 0.25) (layer "F.Cu") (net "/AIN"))
 (segment (start 3.5 6) (end 6.025 6) (width 0.25) (layer "F.Cu") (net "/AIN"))
 (segment (start 31.52 21.825) (end 30.5 21.825) (width 0.25) (layer "F.Cu") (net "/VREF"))
 (via (at 31.52 21.825) (size 0.6) (drill 0.3) (layers "F.Cu" "B.Cu") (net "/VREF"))
 (segment (start 37 11.08) (end 31.52 16.56) (width 0.25) (layer "B.Cu") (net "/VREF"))
 (segment (start 31.52 16.56) (end 31.52 21.825) (width 0.25) (layer "B.Cu") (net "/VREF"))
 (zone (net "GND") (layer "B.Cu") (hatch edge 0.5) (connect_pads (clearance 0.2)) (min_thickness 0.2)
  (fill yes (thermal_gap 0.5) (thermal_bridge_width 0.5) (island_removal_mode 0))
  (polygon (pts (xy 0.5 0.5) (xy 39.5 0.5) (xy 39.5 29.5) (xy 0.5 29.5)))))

